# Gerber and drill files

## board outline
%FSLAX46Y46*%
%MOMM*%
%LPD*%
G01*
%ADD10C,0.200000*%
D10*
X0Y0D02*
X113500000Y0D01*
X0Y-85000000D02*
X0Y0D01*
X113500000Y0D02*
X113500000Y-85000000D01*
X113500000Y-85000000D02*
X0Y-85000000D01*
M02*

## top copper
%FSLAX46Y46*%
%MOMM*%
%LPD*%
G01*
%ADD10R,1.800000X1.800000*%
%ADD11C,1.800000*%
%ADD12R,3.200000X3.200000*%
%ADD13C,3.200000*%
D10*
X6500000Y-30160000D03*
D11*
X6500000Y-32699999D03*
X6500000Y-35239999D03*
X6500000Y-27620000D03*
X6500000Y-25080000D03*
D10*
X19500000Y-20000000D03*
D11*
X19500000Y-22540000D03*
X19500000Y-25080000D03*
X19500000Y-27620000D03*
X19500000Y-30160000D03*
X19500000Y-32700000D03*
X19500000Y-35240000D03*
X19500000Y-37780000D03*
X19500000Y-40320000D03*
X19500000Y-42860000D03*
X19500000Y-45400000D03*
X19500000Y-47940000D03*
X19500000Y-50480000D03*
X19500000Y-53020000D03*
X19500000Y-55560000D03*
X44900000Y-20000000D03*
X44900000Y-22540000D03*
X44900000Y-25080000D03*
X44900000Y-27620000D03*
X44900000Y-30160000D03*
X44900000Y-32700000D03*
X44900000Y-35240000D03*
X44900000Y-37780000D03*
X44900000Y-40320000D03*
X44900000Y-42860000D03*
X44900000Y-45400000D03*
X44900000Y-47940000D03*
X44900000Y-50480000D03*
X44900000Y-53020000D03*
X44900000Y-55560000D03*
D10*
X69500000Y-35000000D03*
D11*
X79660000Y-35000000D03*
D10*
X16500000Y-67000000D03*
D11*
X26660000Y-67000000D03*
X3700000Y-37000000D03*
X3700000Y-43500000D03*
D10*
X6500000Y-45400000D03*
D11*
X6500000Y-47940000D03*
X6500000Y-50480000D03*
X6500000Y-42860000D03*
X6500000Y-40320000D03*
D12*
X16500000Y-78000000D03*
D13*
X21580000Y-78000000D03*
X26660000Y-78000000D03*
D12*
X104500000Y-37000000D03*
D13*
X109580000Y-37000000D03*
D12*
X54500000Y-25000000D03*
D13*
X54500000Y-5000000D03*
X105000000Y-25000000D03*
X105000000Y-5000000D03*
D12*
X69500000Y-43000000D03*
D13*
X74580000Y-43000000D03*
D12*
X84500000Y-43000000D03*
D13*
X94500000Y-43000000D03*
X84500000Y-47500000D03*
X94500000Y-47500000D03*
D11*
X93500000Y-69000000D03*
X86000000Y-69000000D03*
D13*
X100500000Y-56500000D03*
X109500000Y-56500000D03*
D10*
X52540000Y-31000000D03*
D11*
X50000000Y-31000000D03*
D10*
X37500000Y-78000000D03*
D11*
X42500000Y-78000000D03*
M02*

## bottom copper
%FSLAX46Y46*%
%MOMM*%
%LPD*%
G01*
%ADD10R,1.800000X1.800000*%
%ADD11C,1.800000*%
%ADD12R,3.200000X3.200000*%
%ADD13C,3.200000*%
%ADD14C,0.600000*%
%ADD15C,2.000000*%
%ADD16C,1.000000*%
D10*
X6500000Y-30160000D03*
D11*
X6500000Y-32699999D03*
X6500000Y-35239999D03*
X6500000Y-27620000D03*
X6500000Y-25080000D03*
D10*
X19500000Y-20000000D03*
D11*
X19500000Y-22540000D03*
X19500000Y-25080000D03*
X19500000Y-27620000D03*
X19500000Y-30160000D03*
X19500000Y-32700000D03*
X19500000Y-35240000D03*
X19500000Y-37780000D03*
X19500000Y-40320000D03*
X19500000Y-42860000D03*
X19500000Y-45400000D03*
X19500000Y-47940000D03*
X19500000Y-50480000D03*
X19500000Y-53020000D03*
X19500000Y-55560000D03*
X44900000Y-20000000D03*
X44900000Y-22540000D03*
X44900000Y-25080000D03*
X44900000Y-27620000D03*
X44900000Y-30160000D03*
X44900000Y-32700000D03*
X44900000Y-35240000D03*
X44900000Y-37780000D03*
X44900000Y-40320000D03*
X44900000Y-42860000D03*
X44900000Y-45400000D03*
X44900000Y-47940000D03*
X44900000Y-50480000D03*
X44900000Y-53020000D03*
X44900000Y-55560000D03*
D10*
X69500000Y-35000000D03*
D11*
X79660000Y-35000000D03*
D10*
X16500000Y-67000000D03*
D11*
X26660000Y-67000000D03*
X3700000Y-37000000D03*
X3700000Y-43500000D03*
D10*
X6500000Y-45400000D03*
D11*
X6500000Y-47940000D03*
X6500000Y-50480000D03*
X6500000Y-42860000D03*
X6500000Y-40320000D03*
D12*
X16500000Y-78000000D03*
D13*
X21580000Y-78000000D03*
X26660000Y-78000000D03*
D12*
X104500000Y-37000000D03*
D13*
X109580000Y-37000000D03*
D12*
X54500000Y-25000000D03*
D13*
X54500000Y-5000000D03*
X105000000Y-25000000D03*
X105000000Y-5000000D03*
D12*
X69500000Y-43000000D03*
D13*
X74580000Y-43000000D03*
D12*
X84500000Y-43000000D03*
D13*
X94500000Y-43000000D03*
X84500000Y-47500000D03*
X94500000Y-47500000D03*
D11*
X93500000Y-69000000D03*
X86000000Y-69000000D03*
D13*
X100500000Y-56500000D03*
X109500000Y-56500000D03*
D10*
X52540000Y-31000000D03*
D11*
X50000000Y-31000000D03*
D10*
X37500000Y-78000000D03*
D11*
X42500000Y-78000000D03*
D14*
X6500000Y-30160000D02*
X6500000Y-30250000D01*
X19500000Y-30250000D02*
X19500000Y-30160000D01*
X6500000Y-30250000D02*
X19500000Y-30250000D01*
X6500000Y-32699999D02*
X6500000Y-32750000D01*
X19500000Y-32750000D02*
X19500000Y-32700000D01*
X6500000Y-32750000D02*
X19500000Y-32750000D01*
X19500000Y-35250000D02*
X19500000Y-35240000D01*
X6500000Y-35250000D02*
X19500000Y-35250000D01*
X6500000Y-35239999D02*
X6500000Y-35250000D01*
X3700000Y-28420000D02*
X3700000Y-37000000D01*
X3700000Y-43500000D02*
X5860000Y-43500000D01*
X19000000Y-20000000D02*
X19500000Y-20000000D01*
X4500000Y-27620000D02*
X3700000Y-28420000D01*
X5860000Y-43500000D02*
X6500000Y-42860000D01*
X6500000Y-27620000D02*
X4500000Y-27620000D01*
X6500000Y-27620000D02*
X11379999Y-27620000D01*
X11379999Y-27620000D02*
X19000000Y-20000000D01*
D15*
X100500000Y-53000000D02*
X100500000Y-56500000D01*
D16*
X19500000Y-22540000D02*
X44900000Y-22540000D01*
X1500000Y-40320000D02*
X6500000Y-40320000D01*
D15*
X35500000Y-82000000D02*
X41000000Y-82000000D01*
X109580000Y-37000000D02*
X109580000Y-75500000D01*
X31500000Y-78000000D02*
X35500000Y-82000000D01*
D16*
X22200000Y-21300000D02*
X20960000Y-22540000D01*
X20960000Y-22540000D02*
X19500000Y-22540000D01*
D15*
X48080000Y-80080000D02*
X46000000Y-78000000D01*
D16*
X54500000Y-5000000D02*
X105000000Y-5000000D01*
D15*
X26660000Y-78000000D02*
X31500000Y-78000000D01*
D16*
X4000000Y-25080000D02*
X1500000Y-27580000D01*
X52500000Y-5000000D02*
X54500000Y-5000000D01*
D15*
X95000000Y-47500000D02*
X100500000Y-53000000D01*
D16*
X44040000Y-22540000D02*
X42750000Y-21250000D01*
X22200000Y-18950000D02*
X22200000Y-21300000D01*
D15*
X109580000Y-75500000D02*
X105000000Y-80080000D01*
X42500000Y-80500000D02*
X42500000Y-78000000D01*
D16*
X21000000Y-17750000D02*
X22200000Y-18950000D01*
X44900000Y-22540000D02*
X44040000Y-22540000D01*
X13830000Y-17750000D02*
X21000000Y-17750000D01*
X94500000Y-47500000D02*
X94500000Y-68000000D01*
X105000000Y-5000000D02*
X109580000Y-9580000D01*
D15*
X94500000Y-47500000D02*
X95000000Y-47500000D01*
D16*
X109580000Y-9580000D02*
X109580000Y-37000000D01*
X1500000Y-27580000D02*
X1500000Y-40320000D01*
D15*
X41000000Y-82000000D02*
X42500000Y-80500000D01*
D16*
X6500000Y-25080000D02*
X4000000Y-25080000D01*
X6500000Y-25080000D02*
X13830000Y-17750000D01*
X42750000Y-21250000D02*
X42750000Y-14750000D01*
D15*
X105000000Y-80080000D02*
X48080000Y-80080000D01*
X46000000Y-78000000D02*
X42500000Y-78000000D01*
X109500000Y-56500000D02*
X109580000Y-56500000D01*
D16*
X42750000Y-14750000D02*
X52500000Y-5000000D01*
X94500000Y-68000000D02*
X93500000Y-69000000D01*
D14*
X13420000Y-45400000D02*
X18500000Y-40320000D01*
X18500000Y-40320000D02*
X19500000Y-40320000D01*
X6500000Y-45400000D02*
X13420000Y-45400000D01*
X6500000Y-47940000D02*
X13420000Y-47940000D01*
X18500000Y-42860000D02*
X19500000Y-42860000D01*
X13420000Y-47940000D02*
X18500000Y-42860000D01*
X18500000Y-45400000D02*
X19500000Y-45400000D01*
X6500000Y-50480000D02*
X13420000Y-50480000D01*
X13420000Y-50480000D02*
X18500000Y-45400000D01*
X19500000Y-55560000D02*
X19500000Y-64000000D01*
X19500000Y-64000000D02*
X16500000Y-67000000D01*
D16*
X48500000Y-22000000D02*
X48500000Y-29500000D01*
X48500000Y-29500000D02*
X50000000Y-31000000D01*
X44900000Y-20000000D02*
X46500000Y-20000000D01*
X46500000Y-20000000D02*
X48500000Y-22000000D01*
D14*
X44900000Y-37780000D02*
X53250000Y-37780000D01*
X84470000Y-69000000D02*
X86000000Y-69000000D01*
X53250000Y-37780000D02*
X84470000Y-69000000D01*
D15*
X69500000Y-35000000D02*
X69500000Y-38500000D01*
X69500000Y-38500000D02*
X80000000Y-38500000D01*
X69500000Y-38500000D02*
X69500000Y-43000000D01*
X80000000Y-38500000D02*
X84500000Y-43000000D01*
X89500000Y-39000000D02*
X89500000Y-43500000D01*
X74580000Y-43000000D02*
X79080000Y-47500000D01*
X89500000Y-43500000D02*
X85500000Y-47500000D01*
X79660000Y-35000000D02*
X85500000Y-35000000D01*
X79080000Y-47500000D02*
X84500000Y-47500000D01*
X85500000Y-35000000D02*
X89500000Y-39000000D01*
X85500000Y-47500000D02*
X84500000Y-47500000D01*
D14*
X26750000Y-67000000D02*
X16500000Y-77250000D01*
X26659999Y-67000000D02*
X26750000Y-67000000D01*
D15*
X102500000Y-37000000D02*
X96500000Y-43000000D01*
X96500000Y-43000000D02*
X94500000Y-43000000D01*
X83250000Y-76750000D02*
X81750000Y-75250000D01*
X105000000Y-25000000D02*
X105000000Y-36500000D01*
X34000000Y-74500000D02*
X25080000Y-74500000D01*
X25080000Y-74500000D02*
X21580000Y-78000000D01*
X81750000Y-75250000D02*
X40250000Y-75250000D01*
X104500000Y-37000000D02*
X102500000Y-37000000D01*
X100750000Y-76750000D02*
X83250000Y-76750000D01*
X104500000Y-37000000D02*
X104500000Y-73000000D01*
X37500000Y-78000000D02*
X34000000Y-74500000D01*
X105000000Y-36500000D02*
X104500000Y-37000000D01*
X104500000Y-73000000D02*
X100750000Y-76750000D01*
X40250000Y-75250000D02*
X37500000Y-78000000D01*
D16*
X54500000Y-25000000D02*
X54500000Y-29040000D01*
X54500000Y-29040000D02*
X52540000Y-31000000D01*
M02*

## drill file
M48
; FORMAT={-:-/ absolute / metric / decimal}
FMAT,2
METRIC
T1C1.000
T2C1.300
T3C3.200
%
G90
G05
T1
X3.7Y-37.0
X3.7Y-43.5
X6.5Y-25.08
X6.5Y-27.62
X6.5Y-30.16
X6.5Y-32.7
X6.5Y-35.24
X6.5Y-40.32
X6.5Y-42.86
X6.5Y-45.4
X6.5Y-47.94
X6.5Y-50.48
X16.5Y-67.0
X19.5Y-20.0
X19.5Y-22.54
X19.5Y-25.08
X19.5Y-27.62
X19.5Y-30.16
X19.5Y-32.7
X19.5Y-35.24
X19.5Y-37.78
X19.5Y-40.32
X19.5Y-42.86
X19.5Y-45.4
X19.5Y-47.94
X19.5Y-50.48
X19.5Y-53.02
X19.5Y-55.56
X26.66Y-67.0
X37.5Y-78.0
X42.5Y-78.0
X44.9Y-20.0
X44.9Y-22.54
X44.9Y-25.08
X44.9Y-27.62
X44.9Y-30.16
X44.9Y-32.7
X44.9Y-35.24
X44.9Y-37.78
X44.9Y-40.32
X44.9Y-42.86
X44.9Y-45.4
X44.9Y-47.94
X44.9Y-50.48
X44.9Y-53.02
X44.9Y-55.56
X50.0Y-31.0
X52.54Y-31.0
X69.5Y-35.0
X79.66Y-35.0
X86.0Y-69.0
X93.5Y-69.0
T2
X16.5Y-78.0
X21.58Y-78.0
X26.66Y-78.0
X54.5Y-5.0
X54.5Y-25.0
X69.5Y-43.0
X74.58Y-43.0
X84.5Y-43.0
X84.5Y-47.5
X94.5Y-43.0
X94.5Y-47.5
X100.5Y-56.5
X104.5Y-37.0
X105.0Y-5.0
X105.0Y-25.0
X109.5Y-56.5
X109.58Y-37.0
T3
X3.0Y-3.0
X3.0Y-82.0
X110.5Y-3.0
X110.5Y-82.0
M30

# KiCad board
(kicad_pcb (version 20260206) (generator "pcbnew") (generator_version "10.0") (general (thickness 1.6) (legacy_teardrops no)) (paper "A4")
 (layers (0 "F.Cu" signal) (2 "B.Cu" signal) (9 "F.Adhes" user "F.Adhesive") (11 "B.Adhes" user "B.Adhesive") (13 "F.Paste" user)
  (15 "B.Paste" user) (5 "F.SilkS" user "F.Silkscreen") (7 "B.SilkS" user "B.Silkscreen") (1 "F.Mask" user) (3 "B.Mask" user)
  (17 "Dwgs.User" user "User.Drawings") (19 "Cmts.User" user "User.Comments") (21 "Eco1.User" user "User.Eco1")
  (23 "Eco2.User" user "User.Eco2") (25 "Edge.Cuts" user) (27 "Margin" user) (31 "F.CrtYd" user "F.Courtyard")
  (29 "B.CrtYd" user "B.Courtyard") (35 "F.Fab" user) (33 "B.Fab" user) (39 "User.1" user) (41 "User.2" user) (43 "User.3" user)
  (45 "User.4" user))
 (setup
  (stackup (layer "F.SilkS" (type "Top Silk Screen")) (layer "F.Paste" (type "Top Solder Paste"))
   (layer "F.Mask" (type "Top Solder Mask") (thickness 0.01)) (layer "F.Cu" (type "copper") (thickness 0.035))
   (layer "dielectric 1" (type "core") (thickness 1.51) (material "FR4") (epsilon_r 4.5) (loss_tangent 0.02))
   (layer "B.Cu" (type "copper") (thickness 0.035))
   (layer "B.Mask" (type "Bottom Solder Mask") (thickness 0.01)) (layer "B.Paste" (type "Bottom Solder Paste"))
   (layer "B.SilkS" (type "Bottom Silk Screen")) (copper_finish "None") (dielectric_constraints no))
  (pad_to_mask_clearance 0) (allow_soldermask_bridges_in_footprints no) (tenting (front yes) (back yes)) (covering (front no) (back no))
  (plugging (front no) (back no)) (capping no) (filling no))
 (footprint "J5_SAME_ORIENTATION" (layer "F.Cu") (at 6.5 30 -90)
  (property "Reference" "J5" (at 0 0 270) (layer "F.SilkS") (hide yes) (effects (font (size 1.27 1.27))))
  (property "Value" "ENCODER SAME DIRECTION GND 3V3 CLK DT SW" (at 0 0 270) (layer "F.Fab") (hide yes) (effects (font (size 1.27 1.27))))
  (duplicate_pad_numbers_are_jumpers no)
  (pad "1" thru_hole rect (at 0.16 0 270) (size 1.8 1.8) (drill 1) (layers "*.Cu") (remove_unused_layers no) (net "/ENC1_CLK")
   (clearance 0.6) (thermal_bridge_angle 45))
  (pad "2" thru_hole circle (at 2.699999 0 270) (size 1.8 1.8) (drill 1) (layers "*.Cu") (remove_unused_layers no) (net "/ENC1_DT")
   (clearance 0.6))
  (pad "3" thru_hole circle (at 5.239999 0 270) (size 1.8 1.8) (drill 1) (layers "*.Cu") (remove_unused_layers no) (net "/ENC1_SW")
   (clearance 0.6))
  (pad "4" thru_hole circle (at -2.38 0 270) (size 1.8 1.8) (drill 1) (layers "*.Cu") (remove_unused_layers no) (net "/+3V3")
   (clearance 0.6))
  (pad "5" thru_hole circle (at -4.92 0 270) (size 1.8 1.8) (drill 1) (layers "*.Cu") (remove_unused_layers no) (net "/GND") (clearance 0.6)))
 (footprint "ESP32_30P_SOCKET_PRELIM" (layer "F.Cu") (at 19.5 20)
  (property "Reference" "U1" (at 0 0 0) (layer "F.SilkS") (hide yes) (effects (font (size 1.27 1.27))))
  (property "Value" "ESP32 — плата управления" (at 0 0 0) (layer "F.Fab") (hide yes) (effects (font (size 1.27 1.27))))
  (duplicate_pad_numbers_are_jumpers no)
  (pad "1" thru_hole rect (at 0 0) (size 1.8 1.8) (drill 1) (layers "*.Cu") (remove_unused_layers no) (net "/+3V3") (clearance 0.6)
   (thermal_bridge_angle 45))
  (pad "2" thru_hole circle (at 0 2.54) (size 1.8 1.8) (drill 1) (layers "*.Cu") (remove_unused_layers no) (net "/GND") (clearance 0.6))
  (pad "3" thru_hole circle (at 0 5.08) (size 1.8 1.8) (drill 1) (layers "*.Cu") (remove_unused_layers no) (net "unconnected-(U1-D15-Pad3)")
   (clearance 0.6))
  (pad "4" thru_hole circle (at 0 7.62) (size 1.8 1.8) (drill 1) (layers "*.Cu") (remove_unused_layers no) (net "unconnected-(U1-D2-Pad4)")
   (clearance 0.6))
  (pad "5" thru_hole circle (at 0 10.16) (size 1.8 1.8) (drill 1) (layers "*.Cu") (remove_unused_layers no) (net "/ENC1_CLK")
   (clearance 0.6))
  (pad "6" thru_hole circle (at 0 12.7) (size 1.8 1.8) (drill 1) (layers "*.Cu") (remove_unused_layers no) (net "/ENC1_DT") (clearance 0.6))
  (pad "7" thru_hole circle (at 0 15.24) (size 1.8 1.8) (drill 1) (layers "*.Cu") (remove_unused_layers no) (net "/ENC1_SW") (clearance 0.6))
  (pad "8" thru_hole circle (at 0 17.78) (size 1.8 1.8) (drill 1) (layers "*.Cu") (remove_unused_layers no) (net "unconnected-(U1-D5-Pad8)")
   (clearance 0.6))
  (pad "9" thru_hole circle (at 0 20.32) (size 1.8 1.8) (drill 1) (layers "*.Cu") (remove_unused_layers no) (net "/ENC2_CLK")
   (clearance 0.6))
  (pad "10" thru_hole circle (at 0 22.86) (size 1.8 1.8) (drill 1) (layers "*.Cu") (remove_unused_layers no) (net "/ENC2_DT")
   (clearance 0.6))
  (pad "11" thru_hole circle (at 0 25.4) (size 1.8 1.8) (drill 1) (layers "*.Cu") (remove_unused_layers no) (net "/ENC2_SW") (clearance 0.6))
  (pad "12" thru_hole circle (at 0 27.94) (size 1.8 1.8) (drill 1) (layers "*.Cu") (remove_unused_layers no)
   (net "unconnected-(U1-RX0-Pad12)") (clearance 0.6))
  (pad "13" thru_hole circle (at 0 30.48) (size 1.8 1.8) (drill 1) (layers "*.Cu") (remove_unused_layers no)
   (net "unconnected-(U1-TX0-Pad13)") (clearance 0.6))
  (pad "14" thru_hole circle (at 0 33.02) (size 1.8 1.8) (drill 1) (layers "*.Cu") (remove_unused_layers no)
   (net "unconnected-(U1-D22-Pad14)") (clearance 0.6))
  (pad "15" thru_hole circle (at 0 35.56) (size 1.8 1.8) (drill 1) (layers "*.Cu") (remove_unused_layers no) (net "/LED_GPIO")
   (clearance 0.6))
  (pad "16" thru_hole circle (at 25.4 0) (size 1.8 1.8) (drill 1) (layers "*.Cu") (remove_unused_layers no) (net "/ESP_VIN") (clearance 0.6))
  (pad "17" thru_hole circle (at 25.4 2.54) (size 1.8 1.8) (drill 1) (layers "*.Cu") (remove_unused_layers no) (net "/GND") (clearance 0.6))
  (pad "18" thru_hole circle (at 25.4 5.08) (size 1.8 1.8) (drill 1) (layers "*.Cu") (remove_unused_layers no)
   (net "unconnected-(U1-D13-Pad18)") (clearance 0.6))
  (pad "19" thru_hole circle (at 25.4 7.62) (size 1.8 1.8) (drill 1) (layers "*.Cu") (remove_unused_layers no)
   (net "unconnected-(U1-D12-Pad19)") (clearance 0.6))
  (pad "20" thru_hole circle (at 25.4 10.16) (size 1.8 1.8) (drill 1) (layers "*.Cu") (remove_unused_layers no)
   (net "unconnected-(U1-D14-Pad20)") (clearance 0.6))
  (pad "21" thru_hole circle (at 25.4 12.7) (size 1.8 1.8) (drill 1) (layers "*.Cu") (remove_unused_layers no)
   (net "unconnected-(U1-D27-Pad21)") (clearance 0.6))
  (pad "22" thru_hole circle (at 25.4 15.24) (size 1.8 1.8) (drill 1) (layers "*.Cu") (remove_unused_layers no)
   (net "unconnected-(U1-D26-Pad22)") (clearance 0.6))
  (pad "23" thru_hole circle (at 25.4 17.78) (size 1.8 1.8) (drill 1) (layers "*.Cu") (remove_unused_layers no) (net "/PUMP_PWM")
   (clearance 0.6))
  (pad "24" thru_hole circle (at 25.4 20.32) (size 1.8 1.8) (drill 1) (layers "*.Cu") (remove_unused_layers no)
   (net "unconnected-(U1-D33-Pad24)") (clearance 0.6))
  (pad "25" thru_hole circle (at 25.4 22.86) (size 1.8 1.8) (drill 1) (layers "*.Cu") (remove_unused_layers no)
   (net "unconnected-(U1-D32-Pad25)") (clearance 0.6))
  (pad "26" thru_hole circle (at 25.4 25.4) (size 1.8 1.8) (drill 1) (layers "*.Cu") (remove_unused_layers no)
   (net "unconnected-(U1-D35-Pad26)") (clearance 0.6))
  (pad "27" thru_hole circle (at 25.4 27.94) (size 1.8 1.8) (drill 1) (layers "*.Cu") (remove_unused_layers no)
   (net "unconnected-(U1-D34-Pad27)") (clearance 0.6))
  (pad "28" thru_hole circle (at 25.4 30.48) (size 1.8 1.8) (drill 1) (layers "*.Cu") (remove_unused_layers no)
   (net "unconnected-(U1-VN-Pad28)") (clearance 0.6))
  (pad "29" thru_hole circle (at 25.4 33.02) (size 1.8 1.8) (drill 1) (layers "*.Cu") (remove_unused_layers no)
   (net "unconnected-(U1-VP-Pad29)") (clearance 0.6))
  (pad "30" thru_hole circle (at 25.4 35.56) (size 1.8 1.8) (drill 1) (layers "*.Cu") (remove_unused_layers no)
   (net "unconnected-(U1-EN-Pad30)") (clearance 0.6)))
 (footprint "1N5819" (layer "F.Cu") (at 69.5 35)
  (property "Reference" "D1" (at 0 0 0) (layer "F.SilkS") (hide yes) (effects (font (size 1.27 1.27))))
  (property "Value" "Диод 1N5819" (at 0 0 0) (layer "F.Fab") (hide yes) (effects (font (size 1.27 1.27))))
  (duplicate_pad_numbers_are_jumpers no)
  (pad "1" thru_hole rect (at 0 0) (size 1.8 1.8) (drill 1) (layers "*.Cu") (remove_unused_layers no) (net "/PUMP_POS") (clearance 0.6)
   (thermal_bridge_angle 45))
  (pad "2" thru_hole circle (at 10.16 0) (size 1.8 1.8) (drill 1) (layers "*.Cu") (remove_unused_layers no) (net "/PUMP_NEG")
   (clearance 0.6)))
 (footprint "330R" (layer "F.Cu") (at 16.5 67)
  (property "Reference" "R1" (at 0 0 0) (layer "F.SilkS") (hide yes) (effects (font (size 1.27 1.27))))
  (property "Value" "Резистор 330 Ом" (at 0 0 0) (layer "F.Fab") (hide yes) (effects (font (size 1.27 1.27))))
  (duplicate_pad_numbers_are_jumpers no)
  (pad "1" thru_hole rect (at 0 0) (size 1.8 1.8) (drill 1) (layers "*.Cu") (remove_unused_layers no) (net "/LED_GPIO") (clearance 0.6)
   (thermal_bridge_angle 45))
  (pad "2" thru_hole circle (at 10.16 0) (size 1.8 1.8) (drill 1) (layers "*.Cu") (remove_unused_layers no) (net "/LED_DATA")
   (clearance 0.6)))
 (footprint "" (layer "F.Cu") (at 3 82)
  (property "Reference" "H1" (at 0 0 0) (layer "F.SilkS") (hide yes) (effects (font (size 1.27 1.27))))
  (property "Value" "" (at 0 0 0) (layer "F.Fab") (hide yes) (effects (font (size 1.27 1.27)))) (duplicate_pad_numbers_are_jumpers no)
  (pad "" np_thru_hole circle (at 0 0) (size 3.2 3.2) (drill 3.2) (layers "*.Cu") (clearance 0.6)))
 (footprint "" (layer "F.Cu") (at 3.7 37)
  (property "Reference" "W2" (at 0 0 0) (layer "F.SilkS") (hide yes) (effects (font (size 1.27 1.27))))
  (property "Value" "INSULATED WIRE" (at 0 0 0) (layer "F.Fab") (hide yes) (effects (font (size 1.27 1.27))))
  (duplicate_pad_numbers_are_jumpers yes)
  (pad "1" thru_hole circle (at 0 0) (size 1.8 1.8) (drill 1) (layers "*.Cu") (remove_unused_layers no) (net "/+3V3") (clearance 0.6))
  (pad "1" thru_hole circle (at 0 6.5) (size 1.8 1.8) (drill 1) (layers "*.Cu") (remove_unused_layers no) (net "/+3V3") (clearance 0.6)))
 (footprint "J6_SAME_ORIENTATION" (layer "F.Cu") (at 6.5 43 -90)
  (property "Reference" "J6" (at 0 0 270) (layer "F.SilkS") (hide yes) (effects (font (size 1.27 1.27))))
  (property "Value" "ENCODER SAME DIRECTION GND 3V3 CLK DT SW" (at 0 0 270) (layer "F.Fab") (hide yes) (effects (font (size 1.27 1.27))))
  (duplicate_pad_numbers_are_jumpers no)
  (pad "1" thru_hole rect (at 2.4 0 270) (size 1.8 1.8) (drill 1) (layers "*.Cu") (remove_unused_layers no) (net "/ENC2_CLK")
   (clearance 0.6) (thermal_bridge_angle 45))
  (pad "2" thru_hole circle (at 4.94 0 270) (size 1.8 1.8) (drill 1) (layers "*.Cu") (remove_unused_layers no) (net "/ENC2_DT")
   (clearance 0.6))
  (pad "3" thru_hole circle (at 7.48 0 270) (size 1.8 1.8) (drill 1) (layers "*.Cu") (remove_unused_layers no) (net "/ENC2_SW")
   (clearance 0.6))
  (pad "4" thru_hole circle (at -0.14 0 270) (size 1.8 1.8) (drill 1) (layers "*.Cu") (remove_unused_layers no) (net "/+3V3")
   (clearance 0.6))
  (pad "5" thru_hole circle (at -2.68 0 270) (size 1.8 1.8) (drill 1) (layers "*.Cu") (remove_unused_layers no) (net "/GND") (clearance 0.6)))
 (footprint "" (layer "F.Cu") (at 3 3)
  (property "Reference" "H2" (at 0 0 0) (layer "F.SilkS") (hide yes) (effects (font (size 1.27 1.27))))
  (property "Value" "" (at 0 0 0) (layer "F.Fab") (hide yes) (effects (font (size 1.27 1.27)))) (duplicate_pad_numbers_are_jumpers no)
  (pad "" np_thru_hole circle (at 0 0) (size 3.2 3.2) (drill 3.2) (layers "*.Cu") (clearance 0.6)))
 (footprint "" (layer "F.Cu") (at 110.5 82)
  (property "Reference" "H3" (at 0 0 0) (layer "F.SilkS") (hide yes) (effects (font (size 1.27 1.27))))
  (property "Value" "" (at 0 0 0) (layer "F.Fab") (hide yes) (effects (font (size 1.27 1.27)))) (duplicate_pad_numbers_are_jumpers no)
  (pad "" np_thru_hole circle (at 0 0) (size 3.2 3.2) (drill 3.2) (layers "*.Cu") (clearance 0.6)))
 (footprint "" (layer "F.Cu") (at 110.5 3)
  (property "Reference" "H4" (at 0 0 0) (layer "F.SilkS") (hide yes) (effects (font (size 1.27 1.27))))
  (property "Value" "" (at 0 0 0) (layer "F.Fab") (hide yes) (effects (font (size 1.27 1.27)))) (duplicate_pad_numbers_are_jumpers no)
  (pad "" np_thru_hole circle (at 0 0) (size 3.2 3.2) (drill 3.2) (layers "*.Cu") (clearance 0.6)))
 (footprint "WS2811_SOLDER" (layer "F.Cu") (at 16.5 78)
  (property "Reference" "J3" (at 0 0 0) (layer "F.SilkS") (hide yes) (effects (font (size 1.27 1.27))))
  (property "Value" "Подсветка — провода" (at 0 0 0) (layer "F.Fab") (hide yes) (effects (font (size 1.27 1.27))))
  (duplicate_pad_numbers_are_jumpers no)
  (pad "1" thru_hole rect (at 0 0) (size 3.2 3.2) (drill 1.3) (layers "*.Cu") (remove_unused_layers no) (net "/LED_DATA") (clearance 0.6)
   (thermal_bridge_angle 45))
  (pad "2" thru_hole circle (at 5.08 0) (size 3.2 3.2) (drill 1.3) (layers "*.Cu") (remove_unused_layers no) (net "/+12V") (clearance 0.6))
  (pad "3" thru_hole circle (at 10.16 0) (size 3.2 3.2) (drill 1.3) (layers "*.Cu") (remove_unused_layers no) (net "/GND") (clearance 0.6)))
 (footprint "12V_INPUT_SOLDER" (layer "F.Cu") (at 104.5 37)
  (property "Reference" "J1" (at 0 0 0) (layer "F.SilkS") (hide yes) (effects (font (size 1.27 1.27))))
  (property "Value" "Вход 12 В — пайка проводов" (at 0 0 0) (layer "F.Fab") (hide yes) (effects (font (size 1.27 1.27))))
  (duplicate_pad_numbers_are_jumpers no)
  (pad "1" thru_hole rect (at 0 0) (size 3.2 3.2) (drill 1.3) (layers "*.Cu") (remove_unused_layers no) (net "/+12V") (clearance 0.6)
   (thermal_bridge_angle 45))
  (pad "2" thru_hole circle (at 5.08 0) (size 3.2 3.2) (drill 1.3) (layers "*.Cu") (remove_unused_layers no) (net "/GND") (clearance 0.6)))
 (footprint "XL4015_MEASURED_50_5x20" (layer "F.Cu") (at 54.5 25 90)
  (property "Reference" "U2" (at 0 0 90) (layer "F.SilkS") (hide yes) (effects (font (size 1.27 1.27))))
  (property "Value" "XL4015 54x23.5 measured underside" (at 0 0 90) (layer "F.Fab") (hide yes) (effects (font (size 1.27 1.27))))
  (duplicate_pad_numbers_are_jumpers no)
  (pad "1" thru_hole rect (at 0 0 90) (size 3.2 3.2) (drill 1.3) (layers "*.Cu") (remove_unused_layers no) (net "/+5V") (clearance 0.6)
   (thermal_bridge_angle 45))
  (pad "2" thru_hole circle (at 20 0 90) (size 3.2 3.2) (drill 1.3) (layers "*.Cu") (remove_unused_layers no) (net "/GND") (clearance 0.6))
  (pad "3" thru_hole circle (at 0 50.5 90) (size 3.2 3.2) (drill 1.3) (layers "*.Cu") (remove_unused_layers no) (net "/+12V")
   (clearance 0.6))
  (pad "4" thru_hole circle (at 20 50.5 90) (size 3.2 3.2) (drill 1.3) (layers "*.Cu") (remove_unused_layers no) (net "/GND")
   (clearance 0.6)))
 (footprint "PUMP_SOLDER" (layer "F.Cu") (at 69.5 43)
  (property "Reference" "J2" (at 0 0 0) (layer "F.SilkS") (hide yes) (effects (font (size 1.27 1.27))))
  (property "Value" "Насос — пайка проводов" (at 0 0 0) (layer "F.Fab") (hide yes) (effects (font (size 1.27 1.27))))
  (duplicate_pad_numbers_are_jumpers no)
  (pad "1" thru_hole rect (at 0 0) (size 3.2 3.2) (drill 1.3) (layers "*.Cu") (remove_unused_layers no) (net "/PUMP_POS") (clearance 0.6)
   (thermal_bridge_angle 45))
  (pad "2" thru_hole circle (at 5.08 0) (size 3.2 3.2) (drill 1.3) (layers "*.Cu") (remove_unused_layers no) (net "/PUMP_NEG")
   (clearance 0.6)))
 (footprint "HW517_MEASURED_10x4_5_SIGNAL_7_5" (layer "F.Cu") (at 84.5 43)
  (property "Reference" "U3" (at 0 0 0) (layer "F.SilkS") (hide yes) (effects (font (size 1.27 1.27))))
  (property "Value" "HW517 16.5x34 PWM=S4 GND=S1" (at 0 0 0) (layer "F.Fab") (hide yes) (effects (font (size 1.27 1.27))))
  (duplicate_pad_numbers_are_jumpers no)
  (pad "1" thru_hole rect (at 0 0) (size 3.2 3.2) (drill 1.3) (layers "*.Cu") (remove_unused_layers no) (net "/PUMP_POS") (clearance 0.6)
   (thermal_bridge_angle 45))
  (pad "2" thru_hole circle (at 10 0) (size 3.2 3.2) (drill 1.3) (layers "*.Cu") (remove_unused_layers no) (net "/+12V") (clearance 0.6))
  (pad "3" thru_hole circle (at 0 4.5) (size 3.2 3.2) (drill 1.3) (layers "*.Cu") (remove_unused_layers no) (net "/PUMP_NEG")
   (clearance 0.6))
  (pad "4" thru_hole circle (at 10 4.5) (size 3.2 3.2) (drill 1.3) (layers "*.Cu") (remove_unused_layers no) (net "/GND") (clearance 0.6))
  (pad "5" thru_hole circle (at 9 26) (size 1.8 1.8) (drill 1) (layers "*.Cu") (remove_unused_layers no) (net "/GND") (clearance 0.6))
  (pad "6" thru_hole circle (at 1.5 26) (size 1.8 1.8) (drill 1) (layers "*.Cu") (remove_unused_layers no) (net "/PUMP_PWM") (clearance 0.6)))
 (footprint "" (layer "F.Cu") (at 100.5 56.5)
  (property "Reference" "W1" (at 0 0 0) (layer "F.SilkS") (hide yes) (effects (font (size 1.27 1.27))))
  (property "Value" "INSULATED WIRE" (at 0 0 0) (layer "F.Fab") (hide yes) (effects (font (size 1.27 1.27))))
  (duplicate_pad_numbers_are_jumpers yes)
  (pad "1" thru_hole circle (at 0 0) (size 3.2 3.2) (drill 1.3) (layers "*.Cu") (remove_unused_layers no) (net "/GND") (clearance 0.6))
  (pad "1" thru_hole circle (at 9 0) (size 3.2 3.2) (drill 1.3) (layers "*.Cu") (remove_unused_layers no) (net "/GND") (clearance 0.6)))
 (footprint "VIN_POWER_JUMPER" (layer "F.Cu") (at 52.54 31)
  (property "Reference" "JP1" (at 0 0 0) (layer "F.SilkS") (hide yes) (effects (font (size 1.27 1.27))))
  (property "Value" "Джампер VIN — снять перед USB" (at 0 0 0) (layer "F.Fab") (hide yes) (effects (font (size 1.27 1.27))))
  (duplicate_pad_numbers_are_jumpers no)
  (pad "1" thru_hole rect (at 0 0) (size 1.8 1.8) (drill 1) (layers "*.Cu") (remove_unused_layers no) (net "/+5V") (clearance 0.6)
   (thermal_bridge_angle 45))
  (pad "2" thru_hole circle (at -2.54 0) (size 1.8 1.8) (drill 1) (layers "*.Cu") (remove_unused_layers no) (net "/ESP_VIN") (clearance 0.6)))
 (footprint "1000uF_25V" (layer "F.Cu") (at 37.5 78)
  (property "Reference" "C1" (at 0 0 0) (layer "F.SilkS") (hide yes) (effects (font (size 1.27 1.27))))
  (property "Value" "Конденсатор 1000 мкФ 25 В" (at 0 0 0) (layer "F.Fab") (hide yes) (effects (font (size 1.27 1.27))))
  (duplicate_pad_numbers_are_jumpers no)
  (pad "1" thru_hole rect (at 0 0) (size 1.8 1.8) (drill 1) (layers "*.Cu") (remove_unused_layers no) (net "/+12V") (clearance 0.6)
   (thermal_bridge_angle 45))
  (pad "2" thru_hole circle (at 5 0) (size 1.8 1.8) (drill 1) (layers "*.Cu") (remove_unused_layers no) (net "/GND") (clearance 0.6)))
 (gr_line (start 0 0) (end 113.5 0) (stroke (width 0.2) (type default)) (layer "Edge.Cuts"))
 (gr_line (start 0 85) (end 0 0) (stroke (width 0.2) (type default)) (layer "Edge.Cuts"))
 (gr_line (start 113.5 0) (end 113.5 85) (stroke (width 0.2) (type default)) (layer "Edge.Cuts"))
 (gr_line (start 113.5 85) (end 0 85) (stroke (width 0.2) (type default)) (layer "Edge.Cuts"))
 (segment (start 6.5 30.16) (end 6.5 30.25) (width 0.6) (layer "B.Cu") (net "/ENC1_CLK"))
 (segment (start 19.5 30.25) (end 19.5 30.16) (width 0.6) (layer "B.Cu") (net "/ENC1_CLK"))
 (segment (start 6.5 30.25) (end 19.5 30.25) (width 0.6) (layer "B.Cu") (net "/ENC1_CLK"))
 (segment (start 6.5 32.699999) (end 6.5 32.75) (width 0.6) (layer "B.Cu") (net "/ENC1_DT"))
 (segment (start 19.5 32.75) (end 19.5 32.7) (width 0.6) (layer "B.Cu") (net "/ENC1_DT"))
 (segment (start 6.5 32.75) (end 19.5 32.75) (width 0.6) (layer "B.Cu") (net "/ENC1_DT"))
 (segment (start 19.5 35.25) (end 19.5 35.24) (width 0.6) (layer "B.Cu") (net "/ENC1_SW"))
 (segment (start 6.5 35.25) (end 19.5 35.25) (width 0.6) (layer "B.Cu") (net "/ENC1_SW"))
 (segment (start 6.5 35.239999) (end 6.5 35.25) (width 0.6) (layer "B.Cu") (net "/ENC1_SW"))
 (segment (start 3.7 28.42) (end 3.7 37) (width 0.6) (layer "B.Cu") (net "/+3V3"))
 (segment (start 3.7 43.5) (end 5.86 43.5) (width 0.6) (layer "B.Cu") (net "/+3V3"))
 (segment (start 19 20) (end 19.5 20) (width 0.6) (layer "B.Cu") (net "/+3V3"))
 (segment (start 4.5 27.62) (end 3.7 28.42) (width 0.6) (layer "B.Cu") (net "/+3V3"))
 (segment (start 5.86 43.5) (end 6.5 42.86) (width 0.6) (layer "B.Cu") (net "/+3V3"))
 (segment (start 6.5 27.62) (end 4.5 27.62) (width 0.6) (layer "B.Cu") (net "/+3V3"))
 (segment (start 6.5 27.62) (end 11.379999 27.62) (width 0.6) (layer "B.Cu") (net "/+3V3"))
 (segment (start 11.379999 27.62) (end 19 20) (width 0.6) (layer "B.Cu") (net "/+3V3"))
 (segment (start 100.5 53) (end 100.5 56.5) (width 2) (layer "B.Cu") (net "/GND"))
 (segment (start 19.5 22.54) (end 44.9 22.54) (width 1) (layer "B.Cu") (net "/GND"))
 (segment (start 1.5 40.32) (end 6.5 40.32) (width 1) (layer "B.Cu") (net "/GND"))
 (segment (start 35.5 82) (end 41 82) (width 2) (layer "B.Cu") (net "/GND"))
 (segment (start 109.58 37) (end 109.58 75.5) (width 2) (layer "B.Cu") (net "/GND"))
 (segment (start 31.5 78) (end 35.5 82) (width 2) (layer "B.Cu") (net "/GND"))
 (segment (start 22.2 21.3) (end 20.96 22.54) (width 1) (layer "B.Cu") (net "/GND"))
 (segment (start 20.96 22.54) (end 19.5 22.54) (width 1) (layer "B.Cu") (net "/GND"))
 (segment (start 48.08 80.08) (end 46 78) (width 2) (layer "B.Cu") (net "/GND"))
 (segment (start 54.5 5) (end 105 5) (width 1) (layer "B.Cu") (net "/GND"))
 (segment (start 26.66 78) (end 31.5 78) (width 2) (layer "B.Cu") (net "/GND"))
 (segment (start 4 25.08) (end 1.5 27.58) (width 1) (layer "B.Cu") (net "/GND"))
 (segment (start 52.5 5) (end 54.5 5) (width 1) (layer "B.Cu") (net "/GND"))
 (segment (start 95 47.5) (end 100.5 53) (width 2) (layer "B.Cu") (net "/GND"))
 (segment (start 44.04 22.54) (end 42.75 21.25) (width 1) (layer "B.Cu") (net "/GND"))
 (segment (start 22.2 18.95) (end 22.2 21.3) (width 1) (layer "B.Cu") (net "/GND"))
 (segment (start 109.58 75.5) (end 105 80.08) (width 2) (layer "B.Cu") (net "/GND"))
 (segment (start 42.5 80.5) (end 42.5 78) (width 2) (layer "B.Cu") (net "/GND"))
 (segment (start 21 17.75) (end 22.2 18.95) (width 1) (layer "B.Cu") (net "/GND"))
 (segment (start 44.9 22.54) (end 44.04 22.54) (width 1) (layer "B.Cu") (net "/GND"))
 (segment (start 13.83 17.75) (end 21 17.75) (width 1) (layer "B.Cu") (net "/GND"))
 (segment (start 94.5 47.5) (end 94.5 68) (width 1) (layer "B.Cu") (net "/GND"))
 (segment (start 105 5) (end 109.58 9.58) (width 1) (layer "B.Cu") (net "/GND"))
 (segment (start 94.5 47.5) (end 95 47.5) (width 2) (layer "B.Cu") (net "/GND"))
 (segment (start 109.58 9.58) (end 109.58 37) (width 1) (layer "B.Cu") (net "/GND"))
 (segment (start 1.5 27.58) (end 1.5 40.32) (width 1) (layer "B.Cu") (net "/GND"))
 (segment (start 41 82) (end 42.5 80.5) (width 2) (layer "B.Cu") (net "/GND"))
 (segment (start 6.5 25.08) (end 4 25.08) (width 1) (layer "B.Cu") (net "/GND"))
 (segment (start 6.5 25.08) (end 13.83 17.75) (width 1) (layer "B.Cu") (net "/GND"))
 (segment (start 42.75 21.25) (end 42.75 14.75) (width 1) (layer "B.Cu") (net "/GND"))
 (segment (start 105 80.08) (end 48.08 80.08) (width 2) (layer "B.Cu") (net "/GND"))
 (segment (start 46 78) (end 42.5 78) (width 2) (layer "B.Cu") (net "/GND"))
 (segment (start 109.5 56.5) (end 109.58 56.5) (width 2) (layer "B.Cu") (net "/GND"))
 (segment (start 42.75 14.75) (end 52.5 5) (width 1) (layer "B.Cu") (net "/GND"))
 (segment (start 94.5 68) (end 93.5 69) (width 1) (layer "B.Cu") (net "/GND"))
 (segment (start 13.42 45.4) (end 18.5 40.32) (width 0.6) (layer "B.Cu") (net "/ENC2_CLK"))
 (segment (start 18.5 40.32) (end 19.5 40.32) (width 0.6) (layer "B.Cu") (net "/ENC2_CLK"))
 (segment (start 6.5 45.4) (end 13.42 45.4) (width 0.6) (layer "B.Cu") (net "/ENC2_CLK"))
 (segment (start 6.5 47.94) (end 13.42 47.94) (width 0.6) (layer "B.Cu") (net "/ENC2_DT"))
 (segment (start 18.5 42.86) (end 19.5 42.86) (width 0.6) (layer "B.Cu") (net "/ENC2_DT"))
 (segment (start 13.42 47.94) (end 18.5 42.86) (width 0.6) (layer "B.Cu") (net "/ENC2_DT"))
 (segment (start 18.5 45.4) (end 19.5 45.4) (width 0.6) (layer "B.Cu") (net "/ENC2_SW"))
 (segment (start 6.5 50.48) (end 13.42 50.48) (width 0.6) (layer "B.Cu") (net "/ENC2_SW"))
 (segment (start 13.42 50.48) (end 18.5 45.4) (width 0.6) (layer "B.Cu") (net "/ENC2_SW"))
 (segment (start 19.5 55.56) (end 19.5 64) (width 0.6) (layer "B.Cu") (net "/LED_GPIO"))
 (segment (start 19.5 64) (end 16.5 67) (width 0.6) (layer "B.Cu") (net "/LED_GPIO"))
 (segment (start 48.5 22) (end 48.5 29.5) (width 1) (layer "B.Cu") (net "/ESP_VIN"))
 (segment (start 48.5 29.5) (end 50 31) (width 1) (layer "B.Cu") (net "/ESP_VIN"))
 (segment (start 44.9 20) (end 46.5 20) (width 1) (layer "B.Cu") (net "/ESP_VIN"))
 (segment (start 46.5 20) (end 48.5 22) (width 1) (layer "B.Cu") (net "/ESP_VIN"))
 (segment (start 44.9 37.78) (end 53.25 37.78) (width 0.6) (layer "B.Cu") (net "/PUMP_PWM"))
 (segment (start 84.47 69) (end 86 69) (width 0.6) (layer "B.Cu") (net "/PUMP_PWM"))
 (segment (start 53.25 37.78) (end 84.47 69) (width 0.6) (layer "B.Cu") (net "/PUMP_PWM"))
 (segment (start 69.5 35) (end 69.5 38.5) (width 2) (layer "B.Cu") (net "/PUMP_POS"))
 (segment (start 69.5 38.5) (end 80 38.5) (width 2) (layer "B.Cu") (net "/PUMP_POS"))
 (segment (start 69.5 38.5) (end 69.5 43) (width 2) (layer "B.Cu") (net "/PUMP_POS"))
 (segment (start 80 38.5) (end 84.5 43) (width 2) (layer "B.Cu") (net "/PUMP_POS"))
 (segment (start 89.5 39) (end 89.5 43.5) (width 2) (layer "B.Cu") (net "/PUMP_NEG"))
 (segment (start 74.58 43) (end 79.08 47.5) (width 2) (layer "B.Cu") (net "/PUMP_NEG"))
 (segment (start 89.5 43.5) (end 85.5 47.5) (width 2) (layer "B.Cu") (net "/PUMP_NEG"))
 (segment (start 79.66 35) (end 85.5 35) (width 2) (layer "B.Cu") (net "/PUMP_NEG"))
 (segment (start 79.08 47.5) (end 84.5 47.5) (width 2) (layer "B.Cu") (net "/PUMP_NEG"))
 (segment (start 85.5 35) (end 89.5 39) (width 2) (layer "B.Cu") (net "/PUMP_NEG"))
 (segment (start 85.5 47.5) (end 84.5 47.5) (width 2) (layer "B.Cu") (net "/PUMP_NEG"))
 (segment (start 26.75 67) (end 16.5 77.25) (width 0.6) (layer "B.Cu") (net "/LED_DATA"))
 (segment (start 26.659999 67) (end 26.75 67) (width 0.6) (layer "B.Cu") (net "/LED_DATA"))
 (segment (start 102.5 37) (end 96.5 43) (width 2) (layer "B.Cu") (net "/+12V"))
 (segment (start 96.5 43) (end 94.5 43) (width 2) (layer "B.Cu") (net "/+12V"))
 (segment (start 83.25 76.75) (end 81.75 75.25) (width 2) (layer "B.Cu") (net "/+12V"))
 (segment (start 105 25) (end 105 36.5) (width 2) (layer "B.Cu") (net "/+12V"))
 (segment (start 34 74.5) (end 25.08 74.5) (width 2) (layer "B.Cu") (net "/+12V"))
 (segment (start 25.08 74.5) (end 21.58 78) (width 2) (layer "B.Cu") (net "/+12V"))
 (segment (start 81.75 75.25) (end 40.25 75.25) (width 2) (layer "B.Cu") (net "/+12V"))
 (segment (start 104.5 37) (end 102.5 37) (width 2) (layer "B.Cu") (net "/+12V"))
 (segment (start 100.75 76.75) (end 83.25 76.75) (width 2) (layer "B.Cu") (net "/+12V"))
 (segment (start 104.5 37) (end 104.5 73) (width 2) (layer "B.Cu") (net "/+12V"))
 (segment (start 37.5 78) (end 34 74.5) (width 2) (layer "B.Cu") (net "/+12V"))
 (segment (start 105 36.5) (end 104.5 37) (width 2) (layer "B.Cu") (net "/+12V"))
 (segment (start 104.5 73) (end 100.75 76.75) (width 2) (layer "B.Cu") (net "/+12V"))
 (segment (start 40.25 75.25) (end 37.5 78) (width 2) (layer "B.Cu") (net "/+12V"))
 (segment (start 54.5 25) (end 54.5 29.04) (width 1) (layer "B.Cu") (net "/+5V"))
 (segment (start 54.5 29.04) (end 52.54 31) (width 1) (layer "B.Cu") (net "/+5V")))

